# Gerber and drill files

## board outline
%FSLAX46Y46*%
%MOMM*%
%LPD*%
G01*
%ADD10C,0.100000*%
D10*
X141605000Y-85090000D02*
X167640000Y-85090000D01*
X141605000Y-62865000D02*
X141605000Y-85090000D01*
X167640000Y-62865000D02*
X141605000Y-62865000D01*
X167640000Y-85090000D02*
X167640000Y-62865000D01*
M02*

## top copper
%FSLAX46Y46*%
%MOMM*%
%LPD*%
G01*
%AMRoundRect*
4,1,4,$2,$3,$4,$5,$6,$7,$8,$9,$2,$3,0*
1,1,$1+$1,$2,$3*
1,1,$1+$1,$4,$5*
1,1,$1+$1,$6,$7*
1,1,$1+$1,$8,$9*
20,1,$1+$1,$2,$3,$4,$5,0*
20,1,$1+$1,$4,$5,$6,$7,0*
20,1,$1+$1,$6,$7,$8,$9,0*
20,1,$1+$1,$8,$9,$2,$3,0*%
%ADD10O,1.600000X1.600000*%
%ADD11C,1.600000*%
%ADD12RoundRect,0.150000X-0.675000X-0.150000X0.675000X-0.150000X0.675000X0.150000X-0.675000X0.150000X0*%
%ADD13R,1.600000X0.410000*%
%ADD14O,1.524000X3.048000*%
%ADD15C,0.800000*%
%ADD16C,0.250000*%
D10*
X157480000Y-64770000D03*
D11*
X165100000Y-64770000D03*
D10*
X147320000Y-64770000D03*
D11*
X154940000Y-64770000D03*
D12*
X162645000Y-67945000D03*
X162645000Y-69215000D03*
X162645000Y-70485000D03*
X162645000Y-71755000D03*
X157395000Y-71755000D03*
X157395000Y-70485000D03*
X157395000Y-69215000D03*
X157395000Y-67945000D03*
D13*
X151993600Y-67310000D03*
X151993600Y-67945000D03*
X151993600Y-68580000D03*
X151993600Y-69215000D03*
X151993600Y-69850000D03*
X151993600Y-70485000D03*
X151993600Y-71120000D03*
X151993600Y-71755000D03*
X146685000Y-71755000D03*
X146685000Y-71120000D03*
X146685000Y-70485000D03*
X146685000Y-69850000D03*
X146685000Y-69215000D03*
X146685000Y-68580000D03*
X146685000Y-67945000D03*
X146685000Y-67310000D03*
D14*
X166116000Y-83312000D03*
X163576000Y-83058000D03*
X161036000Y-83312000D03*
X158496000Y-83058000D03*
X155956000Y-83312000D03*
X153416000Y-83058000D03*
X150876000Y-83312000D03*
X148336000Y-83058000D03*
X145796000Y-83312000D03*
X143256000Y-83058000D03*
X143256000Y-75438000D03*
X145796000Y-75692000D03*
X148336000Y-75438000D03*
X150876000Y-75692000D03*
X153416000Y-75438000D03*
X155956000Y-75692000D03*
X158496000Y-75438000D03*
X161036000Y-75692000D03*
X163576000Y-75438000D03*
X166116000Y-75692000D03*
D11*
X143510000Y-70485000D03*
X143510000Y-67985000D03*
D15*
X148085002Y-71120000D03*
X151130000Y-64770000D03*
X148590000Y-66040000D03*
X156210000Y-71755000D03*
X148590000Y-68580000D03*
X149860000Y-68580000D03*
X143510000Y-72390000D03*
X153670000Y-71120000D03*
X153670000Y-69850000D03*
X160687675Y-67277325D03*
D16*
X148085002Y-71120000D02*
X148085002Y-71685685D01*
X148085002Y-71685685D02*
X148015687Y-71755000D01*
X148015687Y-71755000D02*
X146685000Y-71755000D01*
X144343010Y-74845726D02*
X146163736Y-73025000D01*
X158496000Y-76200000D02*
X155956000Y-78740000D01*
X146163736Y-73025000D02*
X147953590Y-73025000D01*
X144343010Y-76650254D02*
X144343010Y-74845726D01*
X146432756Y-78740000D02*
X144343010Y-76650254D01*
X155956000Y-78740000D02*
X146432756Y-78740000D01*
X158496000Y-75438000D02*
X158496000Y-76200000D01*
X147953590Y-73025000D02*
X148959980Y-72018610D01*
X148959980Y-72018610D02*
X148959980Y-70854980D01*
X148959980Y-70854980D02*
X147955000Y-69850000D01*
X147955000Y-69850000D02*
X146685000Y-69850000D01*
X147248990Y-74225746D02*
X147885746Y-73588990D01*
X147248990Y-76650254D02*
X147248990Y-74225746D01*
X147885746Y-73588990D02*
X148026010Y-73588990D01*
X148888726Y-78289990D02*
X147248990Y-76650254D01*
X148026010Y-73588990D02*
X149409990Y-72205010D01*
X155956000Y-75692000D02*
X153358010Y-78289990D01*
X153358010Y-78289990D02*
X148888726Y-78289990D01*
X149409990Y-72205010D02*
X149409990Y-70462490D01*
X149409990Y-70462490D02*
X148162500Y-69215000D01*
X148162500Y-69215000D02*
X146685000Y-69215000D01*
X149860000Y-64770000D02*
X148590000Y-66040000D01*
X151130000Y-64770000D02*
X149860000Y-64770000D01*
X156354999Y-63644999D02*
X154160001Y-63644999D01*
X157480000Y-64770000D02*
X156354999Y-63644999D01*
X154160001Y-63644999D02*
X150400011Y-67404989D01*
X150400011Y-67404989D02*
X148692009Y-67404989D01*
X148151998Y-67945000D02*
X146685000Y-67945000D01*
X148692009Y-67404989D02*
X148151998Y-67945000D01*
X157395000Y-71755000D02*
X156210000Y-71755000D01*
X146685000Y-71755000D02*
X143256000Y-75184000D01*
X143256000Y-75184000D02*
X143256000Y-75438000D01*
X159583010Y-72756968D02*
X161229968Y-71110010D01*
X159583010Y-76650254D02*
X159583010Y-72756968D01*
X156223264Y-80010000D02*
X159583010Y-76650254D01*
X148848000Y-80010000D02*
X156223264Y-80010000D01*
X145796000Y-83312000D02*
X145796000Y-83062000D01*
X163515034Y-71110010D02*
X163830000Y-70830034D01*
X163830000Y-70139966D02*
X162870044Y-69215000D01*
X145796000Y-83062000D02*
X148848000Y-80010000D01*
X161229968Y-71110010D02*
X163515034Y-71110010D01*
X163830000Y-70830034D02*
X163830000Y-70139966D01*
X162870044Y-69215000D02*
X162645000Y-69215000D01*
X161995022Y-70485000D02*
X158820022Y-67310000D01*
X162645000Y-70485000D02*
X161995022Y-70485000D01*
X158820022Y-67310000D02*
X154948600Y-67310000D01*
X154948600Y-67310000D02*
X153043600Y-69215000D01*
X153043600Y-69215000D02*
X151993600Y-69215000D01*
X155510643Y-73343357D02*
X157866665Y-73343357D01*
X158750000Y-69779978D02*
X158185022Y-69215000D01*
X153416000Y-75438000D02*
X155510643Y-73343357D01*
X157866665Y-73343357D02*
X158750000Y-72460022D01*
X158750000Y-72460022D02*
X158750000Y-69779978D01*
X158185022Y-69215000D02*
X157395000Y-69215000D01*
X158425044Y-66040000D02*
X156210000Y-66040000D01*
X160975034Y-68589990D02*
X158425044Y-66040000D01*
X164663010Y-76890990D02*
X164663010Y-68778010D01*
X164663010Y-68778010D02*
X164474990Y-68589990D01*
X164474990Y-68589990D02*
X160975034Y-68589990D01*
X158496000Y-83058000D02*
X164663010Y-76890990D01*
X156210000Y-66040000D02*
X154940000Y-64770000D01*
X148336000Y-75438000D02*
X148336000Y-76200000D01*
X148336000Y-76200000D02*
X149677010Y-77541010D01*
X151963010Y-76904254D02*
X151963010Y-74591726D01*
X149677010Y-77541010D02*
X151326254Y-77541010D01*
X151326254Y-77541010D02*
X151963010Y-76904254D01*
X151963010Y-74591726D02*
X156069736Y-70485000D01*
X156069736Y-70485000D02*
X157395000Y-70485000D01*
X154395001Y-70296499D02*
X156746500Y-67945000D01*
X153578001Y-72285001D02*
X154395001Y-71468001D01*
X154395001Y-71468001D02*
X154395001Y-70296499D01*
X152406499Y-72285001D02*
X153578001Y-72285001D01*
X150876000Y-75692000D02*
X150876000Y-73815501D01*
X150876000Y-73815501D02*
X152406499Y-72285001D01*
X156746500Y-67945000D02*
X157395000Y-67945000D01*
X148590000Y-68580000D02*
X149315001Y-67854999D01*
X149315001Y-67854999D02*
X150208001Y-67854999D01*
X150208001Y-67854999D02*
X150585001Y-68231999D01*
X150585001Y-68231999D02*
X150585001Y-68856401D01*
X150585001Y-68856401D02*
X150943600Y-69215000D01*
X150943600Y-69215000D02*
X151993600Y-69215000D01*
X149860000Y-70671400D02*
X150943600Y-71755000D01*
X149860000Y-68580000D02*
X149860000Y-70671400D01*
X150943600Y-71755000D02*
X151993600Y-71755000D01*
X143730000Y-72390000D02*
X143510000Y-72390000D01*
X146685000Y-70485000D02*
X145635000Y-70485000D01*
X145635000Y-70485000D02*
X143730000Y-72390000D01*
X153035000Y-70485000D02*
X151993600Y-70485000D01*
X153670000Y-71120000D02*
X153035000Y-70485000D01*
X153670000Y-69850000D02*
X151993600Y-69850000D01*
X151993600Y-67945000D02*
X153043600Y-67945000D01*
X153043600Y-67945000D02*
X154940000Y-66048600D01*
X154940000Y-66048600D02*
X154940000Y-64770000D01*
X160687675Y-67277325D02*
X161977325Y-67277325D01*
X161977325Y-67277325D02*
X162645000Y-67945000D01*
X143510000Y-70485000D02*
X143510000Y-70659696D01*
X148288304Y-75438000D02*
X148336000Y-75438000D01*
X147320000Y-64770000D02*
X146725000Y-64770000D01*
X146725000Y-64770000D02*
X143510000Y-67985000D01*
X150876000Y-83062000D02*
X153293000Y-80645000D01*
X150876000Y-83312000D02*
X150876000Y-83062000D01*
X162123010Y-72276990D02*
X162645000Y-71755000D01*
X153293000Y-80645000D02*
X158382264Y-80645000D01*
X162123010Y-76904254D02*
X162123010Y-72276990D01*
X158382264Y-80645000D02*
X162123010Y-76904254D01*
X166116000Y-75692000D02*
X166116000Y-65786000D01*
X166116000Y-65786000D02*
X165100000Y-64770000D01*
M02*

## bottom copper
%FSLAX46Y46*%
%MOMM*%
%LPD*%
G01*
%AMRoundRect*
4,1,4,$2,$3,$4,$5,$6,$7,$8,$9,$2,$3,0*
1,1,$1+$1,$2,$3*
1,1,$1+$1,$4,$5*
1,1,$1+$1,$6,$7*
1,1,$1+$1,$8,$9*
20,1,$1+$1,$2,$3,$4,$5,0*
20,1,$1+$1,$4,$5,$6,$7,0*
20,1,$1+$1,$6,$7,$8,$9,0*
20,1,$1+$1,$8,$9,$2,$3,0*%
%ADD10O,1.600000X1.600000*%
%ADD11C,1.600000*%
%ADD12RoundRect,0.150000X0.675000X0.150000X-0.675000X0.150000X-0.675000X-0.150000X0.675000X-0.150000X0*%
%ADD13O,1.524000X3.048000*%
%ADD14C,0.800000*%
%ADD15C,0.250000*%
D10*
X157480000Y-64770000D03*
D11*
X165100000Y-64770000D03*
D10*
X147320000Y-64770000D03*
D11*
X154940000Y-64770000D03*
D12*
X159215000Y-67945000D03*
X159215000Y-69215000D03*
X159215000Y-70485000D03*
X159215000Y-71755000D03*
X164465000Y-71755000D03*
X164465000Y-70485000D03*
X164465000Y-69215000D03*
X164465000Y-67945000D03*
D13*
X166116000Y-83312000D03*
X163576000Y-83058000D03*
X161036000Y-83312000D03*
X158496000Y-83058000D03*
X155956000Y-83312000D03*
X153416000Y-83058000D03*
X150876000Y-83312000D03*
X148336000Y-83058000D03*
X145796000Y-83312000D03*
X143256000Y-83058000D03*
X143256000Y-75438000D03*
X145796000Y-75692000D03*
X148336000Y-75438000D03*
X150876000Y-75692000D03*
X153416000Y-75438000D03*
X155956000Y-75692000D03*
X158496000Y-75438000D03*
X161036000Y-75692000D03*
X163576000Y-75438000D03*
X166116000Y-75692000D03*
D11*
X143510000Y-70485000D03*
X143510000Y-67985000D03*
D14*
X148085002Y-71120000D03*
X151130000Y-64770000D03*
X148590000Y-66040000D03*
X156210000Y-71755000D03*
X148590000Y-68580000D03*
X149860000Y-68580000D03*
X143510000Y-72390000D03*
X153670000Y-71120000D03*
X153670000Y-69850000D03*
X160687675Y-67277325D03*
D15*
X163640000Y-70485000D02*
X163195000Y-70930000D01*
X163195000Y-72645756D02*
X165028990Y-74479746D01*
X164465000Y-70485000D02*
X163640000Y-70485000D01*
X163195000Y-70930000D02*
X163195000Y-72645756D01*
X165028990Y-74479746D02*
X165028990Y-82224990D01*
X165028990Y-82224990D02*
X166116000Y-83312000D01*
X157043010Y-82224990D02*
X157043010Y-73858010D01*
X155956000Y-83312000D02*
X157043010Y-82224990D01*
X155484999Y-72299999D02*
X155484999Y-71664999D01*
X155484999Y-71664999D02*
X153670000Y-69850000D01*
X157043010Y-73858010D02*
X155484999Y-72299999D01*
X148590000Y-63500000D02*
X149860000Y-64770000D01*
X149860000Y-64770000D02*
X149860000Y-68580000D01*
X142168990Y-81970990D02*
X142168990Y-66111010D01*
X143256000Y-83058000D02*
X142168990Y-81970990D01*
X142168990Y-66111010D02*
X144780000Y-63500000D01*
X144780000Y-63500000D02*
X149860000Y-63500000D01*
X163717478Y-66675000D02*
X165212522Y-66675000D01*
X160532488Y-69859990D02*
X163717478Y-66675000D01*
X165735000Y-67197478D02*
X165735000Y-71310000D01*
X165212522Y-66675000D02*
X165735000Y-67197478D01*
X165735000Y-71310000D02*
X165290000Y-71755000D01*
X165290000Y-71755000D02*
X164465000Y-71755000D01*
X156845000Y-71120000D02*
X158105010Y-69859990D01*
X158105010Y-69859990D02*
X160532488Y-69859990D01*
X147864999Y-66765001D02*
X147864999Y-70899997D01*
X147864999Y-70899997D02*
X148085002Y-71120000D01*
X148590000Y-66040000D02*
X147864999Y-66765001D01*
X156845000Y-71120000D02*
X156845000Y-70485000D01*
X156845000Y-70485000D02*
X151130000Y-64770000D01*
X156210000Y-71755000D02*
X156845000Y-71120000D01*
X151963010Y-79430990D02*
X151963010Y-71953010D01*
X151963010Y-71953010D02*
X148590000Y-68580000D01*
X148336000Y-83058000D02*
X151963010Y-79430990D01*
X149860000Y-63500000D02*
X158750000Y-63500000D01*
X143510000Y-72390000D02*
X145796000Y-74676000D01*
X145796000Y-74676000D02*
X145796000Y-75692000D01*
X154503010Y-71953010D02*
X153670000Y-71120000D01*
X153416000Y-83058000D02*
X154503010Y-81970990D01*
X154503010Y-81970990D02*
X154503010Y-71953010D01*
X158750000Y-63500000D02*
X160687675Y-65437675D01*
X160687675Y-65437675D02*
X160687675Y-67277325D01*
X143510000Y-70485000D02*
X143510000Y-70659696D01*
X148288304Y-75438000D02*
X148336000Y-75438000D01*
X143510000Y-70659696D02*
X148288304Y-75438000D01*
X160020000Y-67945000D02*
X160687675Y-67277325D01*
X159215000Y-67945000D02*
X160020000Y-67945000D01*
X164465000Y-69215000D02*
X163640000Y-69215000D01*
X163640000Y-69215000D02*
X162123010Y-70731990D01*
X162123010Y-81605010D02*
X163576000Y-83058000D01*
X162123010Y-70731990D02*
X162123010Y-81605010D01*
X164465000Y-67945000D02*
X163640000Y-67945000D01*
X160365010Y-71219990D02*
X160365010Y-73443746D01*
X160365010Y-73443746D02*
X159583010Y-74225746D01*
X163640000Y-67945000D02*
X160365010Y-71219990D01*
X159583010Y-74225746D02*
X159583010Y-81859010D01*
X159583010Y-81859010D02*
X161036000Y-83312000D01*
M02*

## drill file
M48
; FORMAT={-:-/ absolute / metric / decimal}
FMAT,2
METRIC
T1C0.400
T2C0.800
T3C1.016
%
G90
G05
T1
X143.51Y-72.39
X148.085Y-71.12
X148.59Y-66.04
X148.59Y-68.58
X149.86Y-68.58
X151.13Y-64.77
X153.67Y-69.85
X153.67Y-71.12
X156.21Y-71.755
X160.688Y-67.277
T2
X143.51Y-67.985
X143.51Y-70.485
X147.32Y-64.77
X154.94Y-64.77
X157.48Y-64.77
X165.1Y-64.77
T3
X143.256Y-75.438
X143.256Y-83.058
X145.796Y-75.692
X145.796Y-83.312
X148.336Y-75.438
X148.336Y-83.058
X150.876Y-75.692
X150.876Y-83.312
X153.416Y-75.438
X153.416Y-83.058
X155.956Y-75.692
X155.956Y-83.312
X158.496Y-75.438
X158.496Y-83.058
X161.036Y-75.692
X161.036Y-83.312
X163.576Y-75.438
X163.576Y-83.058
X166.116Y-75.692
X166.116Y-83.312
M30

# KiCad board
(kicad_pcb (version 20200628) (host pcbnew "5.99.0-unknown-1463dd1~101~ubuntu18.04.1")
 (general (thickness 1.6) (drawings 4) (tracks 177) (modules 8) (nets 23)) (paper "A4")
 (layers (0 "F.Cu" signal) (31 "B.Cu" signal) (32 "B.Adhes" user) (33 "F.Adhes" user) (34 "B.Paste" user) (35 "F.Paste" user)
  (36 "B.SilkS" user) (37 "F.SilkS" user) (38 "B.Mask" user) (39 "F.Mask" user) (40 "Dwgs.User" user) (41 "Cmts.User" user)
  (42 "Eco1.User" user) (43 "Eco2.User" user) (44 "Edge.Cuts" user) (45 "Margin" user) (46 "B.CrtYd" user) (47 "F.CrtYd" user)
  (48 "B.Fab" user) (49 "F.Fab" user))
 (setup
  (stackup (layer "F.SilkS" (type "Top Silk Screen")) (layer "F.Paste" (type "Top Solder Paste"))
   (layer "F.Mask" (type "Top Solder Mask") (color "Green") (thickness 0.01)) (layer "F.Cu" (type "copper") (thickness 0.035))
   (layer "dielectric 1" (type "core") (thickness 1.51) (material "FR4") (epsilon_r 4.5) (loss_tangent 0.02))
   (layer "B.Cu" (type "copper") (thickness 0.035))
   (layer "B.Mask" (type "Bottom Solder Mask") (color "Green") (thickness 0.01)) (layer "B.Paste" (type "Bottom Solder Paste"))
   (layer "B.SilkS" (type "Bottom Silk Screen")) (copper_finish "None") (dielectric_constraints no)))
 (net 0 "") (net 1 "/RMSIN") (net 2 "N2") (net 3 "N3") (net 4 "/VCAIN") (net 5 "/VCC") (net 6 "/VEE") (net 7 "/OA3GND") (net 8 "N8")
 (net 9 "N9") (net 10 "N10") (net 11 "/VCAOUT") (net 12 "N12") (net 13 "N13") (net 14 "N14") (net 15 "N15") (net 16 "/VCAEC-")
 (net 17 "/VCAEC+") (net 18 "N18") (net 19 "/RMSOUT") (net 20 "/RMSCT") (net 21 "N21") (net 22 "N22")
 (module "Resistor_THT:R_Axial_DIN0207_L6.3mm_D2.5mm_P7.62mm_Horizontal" (layer "F.Cu") (at 165.1 64.77 180)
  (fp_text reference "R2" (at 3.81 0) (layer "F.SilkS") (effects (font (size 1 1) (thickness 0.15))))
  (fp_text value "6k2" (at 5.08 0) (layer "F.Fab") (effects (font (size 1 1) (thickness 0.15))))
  (pad "2" thru_hole oval (at 7.62 0 180) (size 1.6 1.6) (drill 0.8) (layers *.Cu *.Mask) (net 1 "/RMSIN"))
  (pad "1" thru_hole circle (at 0 0 180) (size 1.6 1.6) (drill 0.8) (layers *.Cu *.Mask) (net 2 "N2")))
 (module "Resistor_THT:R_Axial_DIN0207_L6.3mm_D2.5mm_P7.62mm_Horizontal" (layer "F.Cu") (at 154.94 64.77 180)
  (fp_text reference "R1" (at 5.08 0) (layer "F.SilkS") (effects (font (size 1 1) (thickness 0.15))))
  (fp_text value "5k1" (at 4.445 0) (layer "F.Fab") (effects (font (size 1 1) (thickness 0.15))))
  (pad "2" thru_hole oval (at 7.62 0 180) (size 1.6 1.6) (drill 0.8) (layers *.Cu *.Mask) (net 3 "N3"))
  (pad "1" thru_hole circle (at 0 0 180) (size 1.6 1.6) (drill 0.8) (layers *.Cu *.Mask) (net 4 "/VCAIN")))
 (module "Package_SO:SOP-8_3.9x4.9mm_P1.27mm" (layer "B.Cu") (at 161.84 69.85 180)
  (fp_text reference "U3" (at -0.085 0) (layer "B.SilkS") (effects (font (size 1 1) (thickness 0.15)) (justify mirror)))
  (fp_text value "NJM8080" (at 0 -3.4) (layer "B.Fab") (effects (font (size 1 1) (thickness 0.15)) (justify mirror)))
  (pad "8" smd roundrect (at 2.625 1.905 180) (size 1.65 0.6) (layers "B.Cu" "B.Paste" "B.Mask") (roundrect_rratio 0.25) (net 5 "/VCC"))
  (pad "7" smd roundrect (at 2.625 0.635 180) (size 1.65 0.6) (layers "B.Cu" "B.Paste" "B.Mask") (roundrect_rratio 0.25))
  (pad "6" smd roundrect (at 2.625 -0.635 180) (size 1.65 0.6) (layers "B.Cu" "B.Paste" "B.Mask") (roundrect_rratio 0.25))
  (pad "5" smd roundrect (at 2.625 -1.905 180) (size 1.65 0.6) (layers "B.Cu" "B.Paste" "B.Mask") (roundrect_rratio 0.25))
  (pad "4" smd roundrect (at -2.625 -1.905 180) (size 1.65 0.6) (layers "B.Cu" "B.Paste" "B.Mask") (roundrect_rratio 0.25) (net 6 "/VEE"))
  (pad "3" smd roundrect (at -2.625 -0.635 180) (size 1.65 0.6) (layers "B.Cu" "B.Paste" "B.Mask") (roundrect_rratio 0.25) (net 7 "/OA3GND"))
  (pad "2" smd roundrect (at -2.625 0.635 180) (size 1.65 0.6) (layers "B.Cu" "B.Paste" "B.Mask") (roundrect_rratio 0.25) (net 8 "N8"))
  (pad "1" smd roundrect (at -2.625 1.905 180) (size 1.65 0.6) (layers "B.Cu" "B.Paste" "B.Mask") (roundrect_rratio 0.25) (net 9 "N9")))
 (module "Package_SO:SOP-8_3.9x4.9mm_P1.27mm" (layer "F.Cu") (at 160.02 69.85)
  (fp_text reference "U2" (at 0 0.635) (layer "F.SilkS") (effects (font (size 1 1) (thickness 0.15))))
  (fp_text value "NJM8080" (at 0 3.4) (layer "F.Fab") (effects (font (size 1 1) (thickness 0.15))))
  (pad "8" smd roundrect (at 2.625 -1.905) (size 1.65 0.6) (layers "F.Cu" "F.Paste" "F.Mask") (roundrect_rratio 0.25) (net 5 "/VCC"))
  (pad "7" smd roundrect (at 2.625 -0.635) (size 1.65 0.6) (layers "F.Cu" "F.Paste" "F.Mask") (roundrect_rratio 0.25) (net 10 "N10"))
  (pad "6" smd roundrect (at 2.625 0.635) (size 1.65 0.6) (layers "F.Cu" "F.Paste" "F.Mask") (roundrect_rratio 0.25) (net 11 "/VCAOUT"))
  (pad "5" smd roundrect (at 2.625 1.905) (size 1.65 0.6) (layers "F.Cu" "F.Paste" "F.Mask") (roundrect_rratio 0.25) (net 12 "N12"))
  (pad "4" smd roundrect (at -2.625 1.905) (size 1.65 0.6) (layers "F.Cu" "F.Paste" "F.Mask") (roundrect_rratio 0.25) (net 6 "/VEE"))
  (pad "3" smd roundrect (at -2.625 0.635) (size 1.65 0.6) (layers "F.Cu" "F.Paste" "F.Mask") (roundrect_rratio 0.25) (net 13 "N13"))
  (pad "2" smd roundrect (at -2.625 -0.635) (size 1.65 0.6) (layers "F.Cu" "F.Paste" "F.Mask") (roundrect_rratio 0.25) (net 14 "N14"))
  (pad "1" smd roundrect (at -2.625 -1.905) (size 1.65 0.6) (layers "F.Cu" "F.Paste" "F.Mask") (roundrect_rratio 0.25) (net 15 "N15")))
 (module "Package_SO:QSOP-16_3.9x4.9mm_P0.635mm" (layer "F.Cu") (at 149.3393 69.5325)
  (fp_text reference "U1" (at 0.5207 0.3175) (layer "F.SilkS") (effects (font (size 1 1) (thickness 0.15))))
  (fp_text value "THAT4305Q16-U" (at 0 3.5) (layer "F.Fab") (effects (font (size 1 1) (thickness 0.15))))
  (pad "16" smd rect (at 2.6543 -2.2225) (size 1.6 0.41) (layers "F.Cu" "F.Paste" "F.Mask"))
  (pad "15" smd rect (at 2.6543 -1.5875) (size 1.6 0.41) (layers "F.Cu" "F.Paste" "F.Mask") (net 4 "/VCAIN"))
  (pad "14" smd rect (at 2.6543 -0.9525) (size 1.6 0.41) (layers "F.Cu" "F.Paste" "F.Mask"))
  (pad "13" smd rect (at 2.6543 -0.3175) (size 1.6 0.41) (layers "F.Cu" "F.Paste" "F.Mask") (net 11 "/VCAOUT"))
  (pad "12" smd rect (at 2.6543 0.3175) (size 1.6 0.41) (layers "F.Cu" "F.Paste" "F.Mask") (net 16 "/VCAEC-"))
  (pad "11" smd rect (at 2.6543 0.9525) (size 1.6 0.41) (layers "F.Cu" "F.Paste" "F.Mask") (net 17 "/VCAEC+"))
  (pad "10" smd rect (at 2.6543 1.5875) (size 1.6 0.41) (layers "F.Cu" "F.Paste" "F.Mask"))
  (pad "9" smd rect (at 2.6543 2.2225) (size 1.6 0.41) (layers "F.Cu" "F.Paste" "F.Mask") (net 5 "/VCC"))
  (pad "8" smd rect (at -2.6543 2.2225) (size 1.6 0.41) (layers "F.Cu" "F.Paste" "F.Mask") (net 6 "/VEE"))
  (pad "7" smd rect (at -2.6543 1.5875) (size 1.6 0.41) (layers "F.Cu" "F.Paste" "F.Mask"))
  (pad "6" smd rect (at -2.6543 0.9525) (size 1.6 0.41) (layers "F.Cu" "F.Paste" "F.Mask") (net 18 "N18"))
  (pad "5" smd rect (at -2.6543 0.3175) (size 1.6 0.41) (layers "F.Cu" "F.Paste" "F.Mask") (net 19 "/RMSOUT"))
  (pad "4" smd rect (at -2.6543 -0.3175) (size 1.6 0.41) (layers "F.Cu" "F.Paste" "F.Mask") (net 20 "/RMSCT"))
  (pad "3" smd rect (at -2.6543 -0.9525) (size 1.6 0.41) (layers "F.Cu" "F.Paste" "F.Mask"))
  (pad "2" smd rect (at -2.6543 -1.5875) (size 1.6 0.41) (layers "F.Cu" "F.Paste" "F.Mask") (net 1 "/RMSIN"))
  (pad "1" smd rect (at -2.6543 -2.2225) (size 1.6 0.41) (layers "F.Cu" "F.Paste" "F.Mask")))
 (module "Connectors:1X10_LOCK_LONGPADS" (layer "F.Cu") (at 143.256 83.185)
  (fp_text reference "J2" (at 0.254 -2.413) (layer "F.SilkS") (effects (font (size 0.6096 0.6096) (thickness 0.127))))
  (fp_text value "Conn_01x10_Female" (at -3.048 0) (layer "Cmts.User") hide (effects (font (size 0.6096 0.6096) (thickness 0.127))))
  (pad "10" thru_hole oval (at 22.86 0.127 180) (size 1.524 3.048) (drill 1.016) (layers *.Cu *.Mask) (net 7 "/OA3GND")
   (solder_mask_margin 0.1016))
  (pad "9" thru_hole oval (at 20.32 -0.127 180) (size 1.524 3.048) (drill 1.016) (layers *.Cu *.Mask) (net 8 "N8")
   (solder_mask_margin 0.1016))
  (pad "8" thru_hole oval (at 17.78 0.127 180) (size 1.524 3.048) (drill 1.016) (layers *.Cu *.Mask) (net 9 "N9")
   (solder_mask_margin 0.1016))
  (pad "7" thru_hole oval (at 15.24 -0.127 180) (size 1.524 3.048) (drill 1.016) (layers *.Cu *.Mask) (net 4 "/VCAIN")
   (solder_mask_margin 0.1016))
  (pad "6" thru_hole oval (at 12.7 0.127 180) (size 1.524 3.048) (drill 1.016) (layers *.Cu *.Mask) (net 16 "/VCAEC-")
   (solder_mask_margin 0.1016))
  (pad "5" thru_hole oval (at 10.16 -0.127 180) (size 1.524 3.048) (drill 1.016) (layers *.Cu *.Mask) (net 17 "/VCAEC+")
   (solder_mask_margin 0.1016))
  (pad "4" thru_hole oval (at 7.62 0.127 180) (size 1.524 3.048) (drill 1.016) (layers *.Cu *.Mask) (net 12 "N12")
   (solder_mask_margin 0.1016))
  (pad "3" thru_hole oval (at 5.08 -0.127 180) (size 1.524 3.048) (drill 1.016) (layers *.Cu *.Mask) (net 11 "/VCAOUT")
   (solder_mask_margin 0.1016))
  (pad "2" thru_hole oval (at 2.54 0.127 180) (size 1.524 3.048) (drill 1.016) (layers *.Cu *.Mask) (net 10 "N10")
   (solder_mask_margin 0.1016))
  (pad "1" thru_hole oval (at 0 -0.127 180) (size 1.524 3.048) (drill 1.016) (layers *.Cu *.Mask) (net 5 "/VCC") (solder_mask_margin 0.1016)))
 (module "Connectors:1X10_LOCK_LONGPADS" (layer "F.Cu") (at 166.116 75.565 180)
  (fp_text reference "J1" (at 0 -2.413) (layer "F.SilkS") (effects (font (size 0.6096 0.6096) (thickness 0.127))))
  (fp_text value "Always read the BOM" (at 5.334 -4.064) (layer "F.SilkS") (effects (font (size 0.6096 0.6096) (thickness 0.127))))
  (pad "10" thru_hole oval (at 22.86 0.127) (size 1.524 3.048) (drill 1.016) (layers *.Cu *.Mask) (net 6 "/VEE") (solder_mask_margin 0.1016))
  (pad "9" thru_hole oval (at 20.32 -0.127) (size 1.524 3.048) (drill 1.016) (layers *.Cu *.Mask) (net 18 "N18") (solder_mask_margin 0.1016))
  (pad "8" thru_hole oval (at 17.78 0.127) (size 1.524 3.048) (drill 1.016) (layers *.Cu *.Mask) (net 13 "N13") (solder_mask_margin 0.1016))
  (pad "7" thru_hole oval (at 15.24 -0.127) (size 1.524 3.048) (drill 1.016) (layers *.Cu *.Mask) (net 15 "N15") (solder_mask_margin 0.1016))
  (pad "6" thru_hole oval (at 12.7 0.127) (size 1.524 3.048) (drill 1.016) (layers *.Cu *.Mask) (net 14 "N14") (solder_mask_margin 0.1016))
  (pad "5" thru_hole oval (at 10.16 -0.127) (size 1.524 3.048) (drill 1.016) (layers *.Cu *.Mask) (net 20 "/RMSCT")
   (solder_mask_margin 0.1016))
  (pad "4" thru_hole oval (at 7.62 0.127) (size 1.524 3.048) (drill 1.016) (layers *.Cu *.Mask) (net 19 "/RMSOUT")
   (solder_mask_margin 0.1016))
  (pad "3" thru_hole oval (at 5.08 -0.127) (size 1.524 3.048) (drill 1.016) (layers *.Cu *.Mask) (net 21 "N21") (solder_mask_margin 0.1016))
  (pad "2" thru_hole oval (at 2.54 0.127) (size 1.524 3.048) (drill 1.016) (layers *.Cu *.Mask) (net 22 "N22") (solder_mask_margin 0.1016))
  (pad "1" thru_hole oval (at 0 -0.127) (size 1.524 3.048) (drill 1.016) (layers *.Cu *.Mask) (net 2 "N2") (solder_mask_margin 0.1016)))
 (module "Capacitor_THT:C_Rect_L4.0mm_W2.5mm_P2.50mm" (layer "F.Cu") (at 143.51 70.485 90)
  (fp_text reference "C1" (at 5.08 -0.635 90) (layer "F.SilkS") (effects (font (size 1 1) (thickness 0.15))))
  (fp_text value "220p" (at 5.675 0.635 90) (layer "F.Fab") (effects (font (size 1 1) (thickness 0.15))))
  (pad "1" thru_hole circle (at 0 0 90) (size 1.6 1.6) (drill 0.8) (layers *.Cu *.Mask) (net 13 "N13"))
  (pad "2" thru_hole circle (at 2.5 0 90) (size 1.6 1.6) (drill 0.8) (layers *.Cu *.Mask) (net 3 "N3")))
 (gr_line (start 141.605 85.09) (end 167.64 85.09) (layer "Edge.Cuts") (width 0.1))
 (gr_line (start 141.605 62.865) (end 141.605 85.09) (layer "Edge.Cuts") (width 0.1))
 (gr_line (start 167.64 62.865) (end 141.605 62.865) (layer "Edge.Cuts") (width 0.1))
 (gr_line (start 167.64 85.09) (end 167.64 62.865) (layer "Edge.Cuts") (width 0.1))
 (segment (start 163.64 70.485) (end 163.195 70.93) (width 0.25) (layer "B.Cu") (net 7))
 (segment (start 163.195 72.645756) (end 165.02899 74.479746) (width 0.25) (layer "B.Cu") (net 7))
 (segment (start 164.465 70.485) (end 163.64 70.485) (width 0.25) (layer "B.Cu") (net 7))
 (segment (start 163.195 70.93) (end 163.195 72.645756) (width 0.25) (layer "B.Cu") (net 7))
 (segment (start 165.02899 74.479746) (end 165.02899 82.22499) (width 0.25) (layer "B.Cu") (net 7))
 (segment (start 165.02899 82.22499) (end 166.116 83.312) (width 0.25) (layer "B.Cu") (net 7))
 (segment (start 157.04301 82.22499) (end 157.04301 73.85801) (width 0.25) (layer "B.Cu") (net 16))
 (segment (start 155.956 83.312) (end 157.04301 82.22499) (width 0.25) (layer "B.Cu") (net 16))
 (segment (start 155.484999 72.299999) (end 155.484999 71.664999) (width 0.25) (layer "B.Cu") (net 16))
 (segment (start 155.484999 71.664999) (end 153.67 69.85) (width 0.25) (layer "B.Cu") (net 16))
 (segment (start 157.04301 73.85801) (end 155.484999 72.299999) (width 0.25) (layer "B.Cu") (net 16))
 (segment (start 148.59 63.5) (end 149.86 64.77) (width 0.25) (layer "B.Cu") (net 5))
 (segment (start 149.86 64.77) (end 149.86 68.58) (width 0.25) (layer "B.Cu") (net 5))
 (segment (start 142.16899 81.97099) (end 142.16899 66.11101) (width 0.25) (layer "B.Cu") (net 5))
 (segment (start 143.256 83.058) (end 142.16899 81.97099) (width 0.25) (layer "B.Cu") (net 5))
 (segment (start 142.16899 66.11101) (end 144.78 63.5) (width 0.25) (layer "B.Cu") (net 5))
 (segment (start 144.78 63.5) (end 149.86 63.5) (width 0.25) (layer "B.Cu") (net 5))
 (segment (start 163.717478 66.675) (end 165.212522 66.675) (width 0.25) (layer "B.Cu") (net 6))
 (segment (start 160.532488 69.85999) (end 163.717478 66.675) (width 0.25) (layer "B.Cu") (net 6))
 (segment (start 165.735 67.197478) (end 165.735 71.31) (width 0.25) (layer "B.Cu") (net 6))
 (segment (start 165.212522 66.675) (end 165.735 67.197478) (width 0.25) (layer "B.Cu") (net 6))
 (segment (start 165.735 71.31) (end 165.29 71.755) (width 0.25) (layer "B.Cu") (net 6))
 (segment (start 165.29 71.755) (end 164.465 71.755) (width 0.25) (layer "B.Cu") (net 6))
 (segment (start 156.845 71.12) (end 158.10501 69.85999) (width 0.25) (layer "B.Cu") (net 6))
 (segment (start 158.10501 69.85999) (end 160.532488 69.85999) (width 0.25) (layer "B.Cu") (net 6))
 (segment (start 147.864999 66.765001) (end 147.864999 70.899997) (width 0.25) (layer "B.Cu") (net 6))
 (via (at 148.085002 71.12) (size 0.8) (drill 0.4) (layers "F.Cu" "B.Cu") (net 6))
 (segment (start 147.864999 70.899997) (end 148.085002 71.12) (width 0.25) (layer "B.Cu") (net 6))
 (segment (start 148.59 66.04) (end 147.864999 66.765001) (width 0.25) (layer "B.Cu") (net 6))
 (segment (start 148.085002 71.12) (end 148.085002 71.685685) (width 0.25) (layer "F.Cu") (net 6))
 (segment (start 148.085002 71.685685) (end 148.015687 71.755) (width 0.25) (layer "F.Cu") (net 6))
 (segment (start 148.015687 71.755) (end 146.685 71.755) (width 0.25) (layer "F.Cu") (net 6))
 (segment (start 144.34301 74.845726) (end 146.163736 73.025) (width 0.25) (layer "F.Cu") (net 19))
 (segment (start 158.496 76.2) (end 155.956 78.74) (width 0.25) (layer "F.Cu") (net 19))
 (segment (start 146.163736 73.025) (end 147.95359 73.025) (width 0.25) (layer "F.Cu") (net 19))
 (segment (start 144.34301 76.650254) (end 144.34301 74.845726) (width 0.25) (layer "F.Cu") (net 19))
 (segment (start 146.432756 78.74) (end 144.34301 76.650254) (width 0.25) (layer "F.Cu") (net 19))
 (segment (start 155.956 78.74) (end 146.432756 78.74) (width 0.25) (layer "F.Cu") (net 19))
 (segment (start 158.496 75.438) (end 158.496 76.2) (width 0.25) (layer "F.Cu") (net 19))
 (segment (start 147.95359 73.025) (end 148.95998 72.01861) (width 0.25) (layer "F.Cu") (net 19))
 (segment (start 148.95998 72.01861) (end 148.95998 70.85498) (width 0.25) (layer "F.Cu") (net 19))
 (segment (start 148.95998 70.85498) (end 147.955 69.85) (width 0.25) (layer "F.Cu") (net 19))
 (segment (start 147.955 69.85) (end 146.685 69.85) (width 0.25) (layer "F.Cu") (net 19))
 (segment (start 147.24899 74.225746) (end 147.885746 73.58899) (width 0.25) (layer "F.Cu") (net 20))
 (segment (start 147.24899 76.650254) (end 147.24899 74.225746) (width 0.25) (layer "F.Cu") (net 20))
 (segment (start 147.885746 73.58899) (end 148.02601 73.58899) (width 0.25) (layer "F.Cu") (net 20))
 (segment (start 148.888726 78.28999) (end 147.24899 76.650254) (width 0.25) (layer "F.Cu") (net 20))
 (segment (start 148.02601 73.58899) (end 149.40999 72.20501) (width 0.25) (layer "F.Cu") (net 20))
 (segment (start 155.956 75.692) (end 153.35801 78.28999) (width 0.25) (layer "F.Cu") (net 20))
 (segment (start 153.35801 78.28999) (end 148.888726 78.28999) (width 0.25) (layer "F.Cu") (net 20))
 (segment (start 149.40999 72.20501) (end 149.40999 70.46249) (width 0.25) (layer "F.Cu") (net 20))
 (segment (start 149.40999 70.46249) (end 148.1625 69.215) (width 0.25) (layer "F.Cu") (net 20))
 (segment (start 148.1625 69.215) (end 146.685 69.215) (width 0.25) (layer "F.Cu") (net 20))
 (segment (start 156.845 71.12) (end 156.845 70.485) (width 0.25) (layer "B.Cu") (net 6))
 (via (at 151.13 64.77) (size 0.8) (drill 0.4) (layers "F.Cu" "B.Cu") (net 6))
 (segment (start 156.845 70.485) (end 151.13 64.77) (width 0.25) (layer "B.Cu") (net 6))
 (via (at 148.59 66.04) (size 0.8) (drill 0.4) (layers "F.Cu" "B.Cu") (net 6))
 (segment (start 149.86 64.77) (end 148.59 66.04) (width 0.25) (layer "F.Cu") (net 6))
 (segment (start 156.21 71.755) (end 156.845 71.12) (width 0.25) (layer "B.Cu") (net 6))
 (segment (start 151.13 64.77) (end 149.86 64.77) (width 0.25) (layer "F.Cu") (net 6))
 (segment (start 156.354999 63.644999) (end 154.160001 63.644999) (width 0.25) (layer "F.Cu") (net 1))
 (segment (start 157.48 64.77) (end 156.354999 63.644999) (width 0.25) (layer "F.Cu") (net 1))
 (segment (start 154.160001 63.644999) (end 150.400011 67.404989) (width 0.25) (layer "F.Cu") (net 1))
 (segment (start 150.400011 67.404989) (end 148.692009 67.404989) (width 0.25) (layer "F.Cu") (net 1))
 (segment (start 148.151998 67.945) (end 146.685 67.945) (width 0.25) (layer "F.Cu") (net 1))
 (segment (start 148.692009 67.404989) (end 148.151998 67.945) (width 0.25) (layer "F.Cu") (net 1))
 (via (at 156.21 71.755) (size 0.8) (drill 0.4) (layers "F.Cu" "B.Cu") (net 6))
 (segment (start 157.395 71.755) (end 156.21 71.755) (width 0.25) (layer "F.Cu") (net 6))
 (segment (start 146.685 71.755) (end 143.256 75.184) (width 0.25) (layer "F.Cu") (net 6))
 (segment (start 143.256 75.184) (end 143.256 75.438) (width 0.25) (layer "F.Cu") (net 6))
 (segment (start 159.58301 72.756968) (end 161.229968 71.11001) (width 0.25) (layer "F.Cu") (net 10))
 (segment (start 159.58301 76.650254) (end 159.58301 72.756968) (width 0.25) (layer "F.Cu") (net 10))
 (segment (start 156.223264 80.01) (end 159.58301 76.650254) (width 0.25) (layer "F.Cu") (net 10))
 (segment (start 148.848 80.01) (end 156.223264 80.01) (width 0.25) (layer "F.Cu") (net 10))
 (segment (start 145.796 83.312) (end 145.796 83.062) (width 0.25) (layer "F.Cu") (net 10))
 (segment (start 163.515034 71.11001) (end 163.83 70.830034) (width 0.25) (layer "F.Cu") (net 10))
 (segment (start 163.83 70.139966) (end 162.870044 69.215) (width 0.25) (layer "F.Cu") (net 10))
 (segment (start 145.796 83.062) (end 148.848 80.01) (width 0.25) (layer "F.Cu") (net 10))
 (segment (start 161.229968 71.11001) (end 163.515034 71.11001) (width 0.25) (layer "F.Cu") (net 10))
 (segment (start 163.83 70.830034) (end 163.83 70.139966) (width 0.25) (layer "F.Cu") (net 10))
 (segment (start 162.870044 69.215) (end 162.645 69.215) (width 0.25) (layer "F.Cu") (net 10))
 (segment (start 161.995022 70.485) (end 158.820022 67.31) (width 0.25) (layer "F.Cu") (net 11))
 (segment (start 162.645 70.485) (end 161.995022 70.485) (width 0.25) (layer "F.Cu") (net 11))
 (segment (start 158.820022 67.31) (end 154.9486 67.31) (width 0.25) (layer "F.Cu") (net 11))
 (segment (start 154.9486 67.31) (end 153.0436 69.215) (width 0.25) (layer "F.Cu") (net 11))
 (segment (start 153.0436 69.215) (end 151.9936 69.215) (width 0.25) (layer "F.Cu") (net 11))
 (segment (start 155.510643 73.343357) (end 157.866665 73.343357) (width 0.25) (layer "F.Cu") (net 14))
 (segment (start 158.75 69.779978) (end 158.185022 69.215) (width 0.25) (layer "F.Cu") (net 14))
 (segment (start 153.416 75.438) (end 155.510643 73.343357) (width 0.25) (layer "F.Cu") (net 14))
 (segment (start 157.866665 73.343357) (end 158.75 72.460022) (width 0.25) (layer "F.Cu") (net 14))
 (segment (start 158.75 72.460022) (end 158.75 69.779978) (width 0.25) (layer "F.Cu") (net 14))
 (segment (start 158.185022 69.215) (end 157.395 69.215) (width 0.25) (layer "F.Cu") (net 14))
 (segment (start 158.425044 66.04) (end 156.21 66.04) (width 0.25) (layer "F.Cu") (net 4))
 (segment (start 160.975034 68.58999) (end 158.425044 66.04) (width 0.25) (layer "F.Cu") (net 4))
 (segment (start 164.66301 76.89099) (end 164.66301 68.77801) (width 0.25) (layer "F.Cu") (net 4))
 (segment (start 164.66301 68.77801) (end 164.47499 68.58999) (width 0.25) (layer "F.Cu") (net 4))
 (segment (start 164.47499 68.58999) (end 160.975034 68.58999) (width 0.25) (layer "F.Cu") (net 4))
 (segment (start 158.496 83.058) (end 164.66301 76.89099) (width 0.25) (layer "F.Cu") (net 4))
 (segment (start 156.21 66.04) (end 154.94 64.77) (width 0.25) (layer "F.Cu") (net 4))
 (segment (start 148.336 75.438) (end 148.336 76.2) (width 0.25) (layer "F.Cu") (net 13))
 (segment (start 148.336 76.2) (end 149.67701 77.54101) (width 0.25) (layer "F.Cu") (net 13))
 (segment (start 151.96301 76.904254) (end 151.96301 74.591726) (width 0.25) (layer "F.Cu") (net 13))
 (segment (start 149.67701 77.54101) (end 151.326254 77.54101) (width 0.25) (layer "F.Cu") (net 13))
 (segment (start 151.326254 77.54101) (end 151.96301 76.904254) (width 0.25) (layer "F.Cu") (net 13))
 (segment (start 151.96301 74.591726) (end 156.069736 70.485) (width 0.25) (layer "F.Cu") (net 13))
 (segment (start 156.069736 70.485) (end 157.395 70.485) (width 0.25) (layer "F.Cu") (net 13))
 (segment (start 154.395001 70.296499) (end 156.7465 67.945) (width 0.25) (layer "F.Cu") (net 15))
 (segment (start 153.578001 72.285001) (end 154.395001 71.468001) (width 0.25) (layer "F.Cu") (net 15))
 (segment (start 154.395001 71.468001) (end 154.395001 70.296499) (width 0.25) (layer "F.Cu") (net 15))
 (segment (start 152.406499 72.285001) (end 153.578001 72.285001) (width 0.25) (layer "F.Cu") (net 15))
 (segment (start 150.876 75.692) (end 150.876 73.815501) (width 0.25) (layer "F.Cu") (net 15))
 (segment (start 150.876 73.815501) (end 152.406499 72.285001) (width 0.25) (layer "F.Cu") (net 15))
 (segment (start 156.7465 67.945) (end 157.395 67.945) (width 0.25) (layer "F.Cu") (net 15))
 (segment (start 151.96301 79.43099) (end 151.96301 71.95301) (width 0.25) (layer "B.Cu") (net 11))
 (via (at 148.59 68.58) (size 0.8) (drill 0.4) (layers "F.Cu" "B.Cu") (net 11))
 (segment (start 151.96301 71.95301) (end 148.59 68.58) (width 0.25) (layer "B.Cu") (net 11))
 (segment (start 148.336 83.058) (end 151.96301 79.43099) (width 0.25) (layer "B.Cu") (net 11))
 (segment (start 148.59 68.58) (end 149.315001 67.854999) (width 0.25) (layer "F.Cu") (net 11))
 (segment (start 149.315001 67.854999) (end 150.208001 67.854999) (width 0.25) (layer "F.Cu") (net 11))
 (segment (start 150.208001 67.854999) (end 150.585001 68.231999) (width 0.25) (layer "F.Cu") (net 11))
 (segment (start 150.585001 68.231999) (end 150.585001 68.856401) (width 0.25) (layer "F.Cu") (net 11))
 (segment (start 150.585001 68.856401) (end 150.9436 69.215) (width 0.25) (layer "F.Cu") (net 11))
 (segment (start 150.9436 69.215) (end 151.9936 69.215) (width 0.25) (layer "F.Cu") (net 11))
 (segment (start 149.86 70.6714) (end 150.9436 71.755) (width 0.25) (layer "F.Cu") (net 5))
 (via (at 149.86 68.58) (size 0.8) (drill 0.4) (layers "F.Cu" "B.Cu") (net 5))
 (segment (start 149.86 63.5) (end 158.75 63.5) (width 0.25) (layer "B.Cu") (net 5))
 (segment (start 149.86 68.58) (end 149.86 70.6714) (width 0.25) (layer "F.Cu") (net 5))
 (segment (start 150.9436 71.755) (end 151.9936 71.755) (width 0.25) (layer "F.Cu") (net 5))
 (segment (start 143.73 72.39) (end 143.51 72.39) (width 0.25) (layer "F.Cu") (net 18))
 (via (at 143.51 72.39) (size 0.8) (drill 0.4) (layers "F.Cu" "B.Cu") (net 18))
 (segment (start 146.685 70.485) (end 145.635 70.485) (width 0.25) (layer "F.Cu") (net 18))
 (segment (start 145.635 70.485) (end 143.73 72.39) (width 0.25) (layer "F.Cu") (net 18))
 (segment (start 143.51 72.39) (end 145.796 74.676) (width 0.25) (layer "B.Cu") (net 18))
 (segment (start 145.796 74.676) (end 145.796 75.692) (width 0.25) (layer "B.Cu") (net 18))
 (segment (start 154.50301 71.95301) (end 153.67 71.12) (width 0.25) (layer "B.Cu") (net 17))
 (segment (start 153.416 83.058) (end 154.50301 81.97099) (width 0.25) (layer "B.Cu") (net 17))
 (via (at 153.67 71.12) (size 0.8) (drill 0.4) (layers "F.Cu" "B.Cu") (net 17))
 (segment (start 153.035 70.485) (end 151.9936 70.485) (width 0.25) (layer "F.Cu") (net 17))
 (segment (start 154.50301 81.97099) (end 154.50301 71.95301) (width 0.25) (layer "B.Cu") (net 17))
 (segment (start 153.67 71.12) (end 153.035 70.485) (width 0.25) (layer "F.Cu") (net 17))
 (via (at 153.67 69.85) (size 0.8) (drill 0.4) (layers "F.Cu" "B.Cu") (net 16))
 (segment (start 153.67 69.85) (end 151.9936 69.85) (width 0.25) (layer "F.Cu") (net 16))
 (segment (start 151.9936 67.945) (end 153.0436 67.945) (width 0.25) (layer "F.Cu") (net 4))
 (segment (start 153.0436 67.945) (end 154.94 66.0486) (width 0.25) (layer "F.Cu") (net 4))
 (segment (start 154.94 66.0486) (end 154.94 64.77) (width 0.25) (layer "F.Cu") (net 4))
 (segment (start 158.75 63.5) (end 160.687675 65.437675) (width 0.25) (layer "B.Cu") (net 5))
 (segment (start 160.687675 65.437675) (end 160.687675 67.277325) (width 0.25) (layer "B.Cu") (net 5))
 (segment (start 143.51 70.485) (end 143.51 70.659696) (width 0.25) (layer "B.Cu") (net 13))
 (segment (start 148.288304 75.438) (end 148.336 75.438) (width 0.25) (layer "B.Cu") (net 13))
 (segment (start 143.51 70.659696) (end 148.288304 75.438) (width 0.25) (layer "B.Cu") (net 13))
 (via (at 160.687675 67.277325) (size 0.8) (drill 0.4) (layers "F.Cu" "B.Cu") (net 5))
 (segment (start 160.02 67.945) (end 160.687675 67.277325) (width 0.25) (layer "B.Cu") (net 5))
 (segment (start 159.215 67.945) (end 160.02 67.945) (width 0.25) (layer "B.Cu") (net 5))
 (segment (start 160.687675 67.277325) (end 161.977325 67.277325) (width 0.25) (layer "F.Cu") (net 5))
 (segment (start 161.977325 67.277325) (end 162.645 67.945) (width 0.25) (layer "F.Cu") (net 5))
 (segment (start 143.51 70.485) (end 143.51 70.659696) (width 0.25) (layer "F.Cu") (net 13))
 (segment (start 148.288304 75.438) (end 148.336 75.438) (width 0.25) (layer "F.Cu") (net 13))
 (segment (start 147.32 64.77) (end 146.725 64.77) (width 0.25) (layer "F.Cu") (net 3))
 (segment (start 146.725 64.77) (end 143.51 67.985) (width 0.25) (layer "F.Cu") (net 3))
 (segment (start 150.876 83.062) (end 153.293 80.645) (width 0.25) (layer "F.Cu") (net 12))
 (segment (start 150.876 83.312) (end 150.876 83.062) (width 0.25) (layer "F.Cu") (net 12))
 (segment (start 162.12301 72.27699) (end 162.645 71.755) (width 0.25) (layer "F.Cu") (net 12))
 (segment (start 153.293 80.645) (end 158.382264 80.645) (width 0.25) (layer "F.Cu") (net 12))
 (segment (start 162.12301 76.904254) (end 162.12301 72.27699) (width 0.25) (layer "F.Cu") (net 12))
 (segment (start 158.382264 80.645) (end 162.12301 76.904254) (width 0.25) (layer "F.Cu") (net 12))
 (segment (start 164.465 69.215) (end 163.64 69.215) (width 0.25) (layer "B.Cu") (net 8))
 (segment (start 163.64 69.215) (end 162.12301 70.73199) (width 0.25) (layer "B.Cu") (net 8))
 (segment (start 162.12301 81.60501) (end 163.576 83.058) (width 0.25) (layer "B.Cu") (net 8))
 (segment (start 162.12301 70.73199) (end 162.12301 81.60501) (width 0.25) (layer "B.Cu") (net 8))
 (segment (start 164.465 67.945) (end 163.64 67.945) (width 0.25) (layer "B.Cu") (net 9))
 (segment (start 160.36501 71.21999) (end 160.36501 73.443746) (width 0.25) (layer "B.Cu") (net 9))
 (segment (start 160.36501 73.443746) (end 159.58301 74.225746) (width 0.25) (layer "B.Cu") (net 9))
 (segment (start 163.64 67.945) (end 160.36501 71.21999) (width 0.25) (layer "B.Cu") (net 9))
 (segment (start 159.58301 74.225746) (end 159.58301 81.85901) (width 0.25) (layer "B.Cu") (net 9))
 (segment (start 159.58301 81.85901) (end 161.036 83.312) (width 0.25) (layer "B.Cu") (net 9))
 (segment (start 166.116 75.692) (end 166.116 65.786) (width 0.25) (layer "F.Cu") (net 2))
 (segment (start 166.116 65.786) (end 165.1 64.77) (width 0.25) (layer "F.Cu") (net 2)))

